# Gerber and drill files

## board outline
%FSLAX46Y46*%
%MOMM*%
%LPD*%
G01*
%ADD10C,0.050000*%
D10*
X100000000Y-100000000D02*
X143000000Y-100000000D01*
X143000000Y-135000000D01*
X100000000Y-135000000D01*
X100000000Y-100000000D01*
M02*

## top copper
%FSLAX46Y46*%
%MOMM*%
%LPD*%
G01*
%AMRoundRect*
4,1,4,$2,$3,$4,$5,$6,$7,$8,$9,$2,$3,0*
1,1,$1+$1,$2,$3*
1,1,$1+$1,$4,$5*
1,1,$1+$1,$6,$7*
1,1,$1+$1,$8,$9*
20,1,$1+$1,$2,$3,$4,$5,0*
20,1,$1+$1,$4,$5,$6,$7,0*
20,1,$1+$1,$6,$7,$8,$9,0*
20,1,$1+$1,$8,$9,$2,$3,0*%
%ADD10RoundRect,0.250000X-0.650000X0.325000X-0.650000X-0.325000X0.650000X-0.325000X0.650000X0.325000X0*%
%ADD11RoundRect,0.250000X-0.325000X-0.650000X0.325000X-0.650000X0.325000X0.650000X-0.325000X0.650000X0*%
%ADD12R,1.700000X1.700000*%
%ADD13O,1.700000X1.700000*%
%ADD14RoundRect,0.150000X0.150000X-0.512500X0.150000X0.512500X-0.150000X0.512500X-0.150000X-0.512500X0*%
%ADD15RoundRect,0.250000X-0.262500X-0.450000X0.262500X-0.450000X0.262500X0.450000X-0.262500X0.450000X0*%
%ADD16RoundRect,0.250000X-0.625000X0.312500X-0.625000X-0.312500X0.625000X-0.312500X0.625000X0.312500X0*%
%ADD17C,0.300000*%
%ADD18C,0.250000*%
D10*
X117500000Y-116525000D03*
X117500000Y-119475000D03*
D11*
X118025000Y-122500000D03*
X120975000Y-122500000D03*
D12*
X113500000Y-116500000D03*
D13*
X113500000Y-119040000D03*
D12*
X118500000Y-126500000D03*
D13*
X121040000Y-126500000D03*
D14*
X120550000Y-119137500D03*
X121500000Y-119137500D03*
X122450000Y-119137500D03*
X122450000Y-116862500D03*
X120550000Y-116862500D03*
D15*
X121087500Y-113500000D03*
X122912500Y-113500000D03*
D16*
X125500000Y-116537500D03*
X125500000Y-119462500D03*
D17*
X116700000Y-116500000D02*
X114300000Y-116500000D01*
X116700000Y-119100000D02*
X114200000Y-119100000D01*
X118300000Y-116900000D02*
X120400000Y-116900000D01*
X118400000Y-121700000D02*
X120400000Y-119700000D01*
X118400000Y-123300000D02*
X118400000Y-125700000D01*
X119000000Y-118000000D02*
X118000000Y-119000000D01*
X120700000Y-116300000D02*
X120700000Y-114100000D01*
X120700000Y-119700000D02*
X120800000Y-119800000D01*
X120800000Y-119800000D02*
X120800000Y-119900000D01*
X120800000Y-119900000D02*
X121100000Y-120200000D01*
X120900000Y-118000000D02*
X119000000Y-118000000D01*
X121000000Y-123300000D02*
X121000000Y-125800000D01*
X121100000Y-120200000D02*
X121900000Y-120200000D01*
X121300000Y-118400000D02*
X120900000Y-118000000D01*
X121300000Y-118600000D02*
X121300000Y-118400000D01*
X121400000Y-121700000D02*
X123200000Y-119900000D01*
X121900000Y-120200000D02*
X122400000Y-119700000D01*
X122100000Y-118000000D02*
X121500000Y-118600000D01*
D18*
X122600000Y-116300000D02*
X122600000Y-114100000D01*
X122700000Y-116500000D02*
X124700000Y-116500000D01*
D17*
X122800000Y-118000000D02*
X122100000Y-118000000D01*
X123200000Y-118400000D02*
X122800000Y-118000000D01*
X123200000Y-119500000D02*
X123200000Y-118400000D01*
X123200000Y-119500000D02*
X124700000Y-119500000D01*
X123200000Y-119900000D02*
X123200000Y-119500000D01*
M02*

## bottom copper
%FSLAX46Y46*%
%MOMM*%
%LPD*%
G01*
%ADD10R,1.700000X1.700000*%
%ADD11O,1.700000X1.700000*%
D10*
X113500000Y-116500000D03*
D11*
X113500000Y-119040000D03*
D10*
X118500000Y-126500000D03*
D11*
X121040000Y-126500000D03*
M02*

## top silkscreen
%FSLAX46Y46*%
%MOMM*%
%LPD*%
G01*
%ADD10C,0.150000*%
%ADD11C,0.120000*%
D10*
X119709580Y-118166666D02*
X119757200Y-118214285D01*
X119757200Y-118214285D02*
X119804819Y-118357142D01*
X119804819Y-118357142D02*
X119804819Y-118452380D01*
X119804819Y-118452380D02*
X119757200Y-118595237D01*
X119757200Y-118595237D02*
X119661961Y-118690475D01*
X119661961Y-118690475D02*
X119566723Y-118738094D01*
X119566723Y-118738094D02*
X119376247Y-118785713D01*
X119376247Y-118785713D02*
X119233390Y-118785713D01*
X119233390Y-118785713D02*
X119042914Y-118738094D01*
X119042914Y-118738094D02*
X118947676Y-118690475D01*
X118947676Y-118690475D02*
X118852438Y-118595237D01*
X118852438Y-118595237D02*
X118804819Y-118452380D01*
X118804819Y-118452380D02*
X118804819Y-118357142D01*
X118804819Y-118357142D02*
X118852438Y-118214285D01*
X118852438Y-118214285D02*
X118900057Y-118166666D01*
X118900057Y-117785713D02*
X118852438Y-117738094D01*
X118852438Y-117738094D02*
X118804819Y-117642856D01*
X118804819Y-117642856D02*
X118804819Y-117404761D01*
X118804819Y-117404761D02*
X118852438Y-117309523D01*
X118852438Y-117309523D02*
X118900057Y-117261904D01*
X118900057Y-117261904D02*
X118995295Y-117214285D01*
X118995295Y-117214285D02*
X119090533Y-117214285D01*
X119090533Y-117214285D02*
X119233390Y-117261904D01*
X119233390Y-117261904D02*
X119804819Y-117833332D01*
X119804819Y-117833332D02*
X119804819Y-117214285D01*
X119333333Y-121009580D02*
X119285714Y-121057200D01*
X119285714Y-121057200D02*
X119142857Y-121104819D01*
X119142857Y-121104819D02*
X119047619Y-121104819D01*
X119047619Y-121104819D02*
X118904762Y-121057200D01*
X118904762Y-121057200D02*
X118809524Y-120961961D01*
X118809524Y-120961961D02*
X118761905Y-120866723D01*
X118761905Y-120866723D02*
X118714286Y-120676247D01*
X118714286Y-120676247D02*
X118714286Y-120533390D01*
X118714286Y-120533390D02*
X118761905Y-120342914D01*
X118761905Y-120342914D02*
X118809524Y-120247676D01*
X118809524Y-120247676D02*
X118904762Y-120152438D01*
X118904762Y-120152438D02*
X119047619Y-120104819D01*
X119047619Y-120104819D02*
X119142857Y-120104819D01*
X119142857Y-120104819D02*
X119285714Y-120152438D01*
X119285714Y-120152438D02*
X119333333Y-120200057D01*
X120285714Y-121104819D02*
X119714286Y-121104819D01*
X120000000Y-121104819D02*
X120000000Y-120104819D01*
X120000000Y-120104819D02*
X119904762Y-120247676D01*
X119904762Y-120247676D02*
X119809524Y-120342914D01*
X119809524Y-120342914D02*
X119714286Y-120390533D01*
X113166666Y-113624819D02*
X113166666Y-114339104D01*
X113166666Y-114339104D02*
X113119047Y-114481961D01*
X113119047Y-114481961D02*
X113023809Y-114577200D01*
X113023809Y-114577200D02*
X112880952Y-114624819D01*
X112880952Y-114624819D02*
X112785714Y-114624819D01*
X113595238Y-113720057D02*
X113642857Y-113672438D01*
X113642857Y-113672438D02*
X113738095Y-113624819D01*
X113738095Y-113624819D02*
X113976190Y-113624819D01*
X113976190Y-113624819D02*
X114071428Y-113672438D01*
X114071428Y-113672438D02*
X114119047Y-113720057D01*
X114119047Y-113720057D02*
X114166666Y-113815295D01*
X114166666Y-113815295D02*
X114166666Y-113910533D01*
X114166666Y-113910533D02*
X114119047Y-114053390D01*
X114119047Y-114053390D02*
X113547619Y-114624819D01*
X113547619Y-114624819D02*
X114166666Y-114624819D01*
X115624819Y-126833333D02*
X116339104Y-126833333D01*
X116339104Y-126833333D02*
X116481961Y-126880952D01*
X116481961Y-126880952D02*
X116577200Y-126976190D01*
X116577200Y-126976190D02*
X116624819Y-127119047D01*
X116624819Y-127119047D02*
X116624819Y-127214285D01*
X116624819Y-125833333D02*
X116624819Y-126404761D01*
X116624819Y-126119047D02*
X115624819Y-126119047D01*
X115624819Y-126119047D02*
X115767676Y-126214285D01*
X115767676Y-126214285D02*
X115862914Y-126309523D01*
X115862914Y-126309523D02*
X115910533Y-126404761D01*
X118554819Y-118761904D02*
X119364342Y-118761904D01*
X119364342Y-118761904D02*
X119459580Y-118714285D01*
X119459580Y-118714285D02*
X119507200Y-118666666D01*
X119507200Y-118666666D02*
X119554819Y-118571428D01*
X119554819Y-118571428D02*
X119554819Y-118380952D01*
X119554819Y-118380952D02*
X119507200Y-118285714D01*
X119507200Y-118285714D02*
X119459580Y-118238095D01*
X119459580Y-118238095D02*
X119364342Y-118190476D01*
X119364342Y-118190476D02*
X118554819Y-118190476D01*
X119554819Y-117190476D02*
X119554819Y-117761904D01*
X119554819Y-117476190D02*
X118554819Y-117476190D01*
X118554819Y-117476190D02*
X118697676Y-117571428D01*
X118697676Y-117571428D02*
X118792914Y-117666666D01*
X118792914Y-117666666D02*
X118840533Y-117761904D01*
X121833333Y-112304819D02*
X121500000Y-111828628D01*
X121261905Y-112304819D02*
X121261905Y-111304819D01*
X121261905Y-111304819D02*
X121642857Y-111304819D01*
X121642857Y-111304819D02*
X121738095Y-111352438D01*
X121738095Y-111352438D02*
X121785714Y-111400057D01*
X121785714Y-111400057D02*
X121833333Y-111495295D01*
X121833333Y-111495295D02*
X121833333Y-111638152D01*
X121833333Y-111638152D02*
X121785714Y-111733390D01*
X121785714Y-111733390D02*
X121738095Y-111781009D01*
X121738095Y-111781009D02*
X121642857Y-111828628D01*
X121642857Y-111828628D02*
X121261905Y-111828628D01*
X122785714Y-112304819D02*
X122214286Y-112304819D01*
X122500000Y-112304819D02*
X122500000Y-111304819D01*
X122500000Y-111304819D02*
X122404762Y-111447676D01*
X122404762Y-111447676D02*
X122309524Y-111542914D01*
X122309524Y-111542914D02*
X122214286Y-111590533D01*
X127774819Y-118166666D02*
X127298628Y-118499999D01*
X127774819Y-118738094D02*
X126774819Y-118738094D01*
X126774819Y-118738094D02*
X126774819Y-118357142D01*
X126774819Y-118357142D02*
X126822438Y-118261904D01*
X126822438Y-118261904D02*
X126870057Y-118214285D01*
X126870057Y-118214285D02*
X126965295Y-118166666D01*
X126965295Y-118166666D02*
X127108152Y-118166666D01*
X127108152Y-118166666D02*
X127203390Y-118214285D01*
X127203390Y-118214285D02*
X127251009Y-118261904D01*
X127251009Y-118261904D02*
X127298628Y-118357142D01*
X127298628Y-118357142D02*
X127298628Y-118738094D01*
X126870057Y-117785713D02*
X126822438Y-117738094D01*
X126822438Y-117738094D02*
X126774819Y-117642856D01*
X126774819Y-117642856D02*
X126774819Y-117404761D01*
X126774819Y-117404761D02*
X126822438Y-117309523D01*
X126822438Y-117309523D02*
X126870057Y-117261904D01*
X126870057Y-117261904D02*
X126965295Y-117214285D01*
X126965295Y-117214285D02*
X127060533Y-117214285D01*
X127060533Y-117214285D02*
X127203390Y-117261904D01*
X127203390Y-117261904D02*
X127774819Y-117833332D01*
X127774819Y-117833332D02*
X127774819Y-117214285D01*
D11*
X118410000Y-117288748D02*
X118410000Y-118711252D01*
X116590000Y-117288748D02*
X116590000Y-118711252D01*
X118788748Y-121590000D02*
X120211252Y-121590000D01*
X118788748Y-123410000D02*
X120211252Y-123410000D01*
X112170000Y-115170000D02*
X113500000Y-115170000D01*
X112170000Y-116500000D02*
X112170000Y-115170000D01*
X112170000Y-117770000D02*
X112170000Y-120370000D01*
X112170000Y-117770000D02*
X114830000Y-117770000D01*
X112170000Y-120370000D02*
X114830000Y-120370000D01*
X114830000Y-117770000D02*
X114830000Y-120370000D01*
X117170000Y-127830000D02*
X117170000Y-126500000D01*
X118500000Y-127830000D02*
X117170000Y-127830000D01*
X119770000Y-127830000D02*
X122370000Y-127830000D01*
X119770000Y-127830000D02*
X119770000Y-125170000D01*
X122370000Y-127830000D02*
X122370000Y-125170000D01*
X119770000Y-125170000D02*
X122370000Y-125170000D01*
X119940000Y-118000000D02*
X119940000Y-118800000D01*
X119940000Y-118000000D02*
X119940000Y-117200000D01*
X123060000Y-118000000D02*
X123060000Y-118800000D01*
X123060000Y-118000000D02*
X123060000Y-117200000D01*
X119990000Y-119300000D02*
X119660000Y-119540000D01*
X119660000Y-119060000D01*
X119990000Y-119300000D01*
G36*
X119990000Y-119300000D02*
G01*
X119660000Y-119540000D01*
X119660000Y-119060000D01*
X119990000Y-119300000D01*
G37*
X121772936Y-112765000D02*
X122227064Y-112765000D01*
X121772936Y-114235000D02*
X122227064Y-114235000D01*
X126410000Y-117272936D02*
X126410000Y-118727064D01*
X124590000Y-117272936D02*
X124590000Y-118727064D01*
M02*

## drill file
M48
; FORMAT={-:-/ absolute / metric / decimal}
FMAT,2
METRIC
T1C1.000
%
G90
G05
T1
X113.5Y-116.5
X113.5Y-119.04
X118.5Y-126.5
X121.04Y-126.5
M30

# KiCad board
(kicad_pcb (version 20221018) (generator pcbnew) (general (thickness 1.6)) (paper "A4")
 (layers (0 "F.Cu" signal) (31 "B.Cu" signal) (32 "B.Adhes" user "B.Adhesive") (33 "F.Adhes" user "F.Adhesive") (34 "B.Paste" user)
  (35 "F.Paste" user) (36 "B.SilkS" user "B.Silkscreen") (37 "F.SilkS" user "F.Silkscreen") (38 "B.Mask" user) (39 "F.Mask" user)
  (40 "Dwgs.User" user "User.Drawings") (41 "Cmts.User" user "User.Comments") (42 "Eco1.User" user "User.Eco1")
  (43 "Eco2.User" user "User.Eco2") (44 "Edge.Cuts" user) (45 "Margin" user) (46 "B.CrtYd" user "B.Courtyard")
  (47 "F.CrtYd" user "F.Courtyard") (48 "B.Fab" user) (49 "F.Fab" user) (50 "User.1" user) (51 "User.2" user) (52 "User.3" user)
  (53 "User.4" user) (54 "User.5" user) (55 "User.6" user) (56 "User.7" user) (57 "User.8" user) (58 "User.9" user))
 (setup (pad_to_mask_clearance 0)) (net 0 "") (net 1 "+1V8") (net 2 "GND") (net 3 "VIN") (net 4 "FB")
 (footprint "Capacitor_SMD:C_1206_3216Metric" (layer "F.Cu") (at 117.5 118 -90)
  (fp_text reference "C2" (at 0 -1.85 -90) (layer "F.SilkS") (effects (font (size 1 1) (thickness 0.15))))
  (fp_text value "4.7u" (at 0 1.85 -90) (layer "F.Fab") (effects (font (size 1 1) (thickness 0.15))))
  (fp_line (start -0.711252 -0.91) (end 0.711252 -0.91) (stroke (width 0.12) (type solid)) (layer "F.SilkS"))
  (fp_line (start -0.711252 0.91) (end 0.711252 0.91) (stroke (width 0.12) (type solid)) (layer "F.SilkS"))
  (pad "1" smd roundrect (at -1.475 0 270) (size 1.15 1.8) (layers "F.Cu" "F.Paste" "F.Mask") (roundrect_rratio 0.217391) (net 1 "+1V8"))
  (pad "2" smd roundrect (at 1.475 0 270) (size 1.15 1.8) (layers "F.Cu" "F.Paste" "F.Mask") (roundrect_rratio 0.217391) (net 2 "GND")))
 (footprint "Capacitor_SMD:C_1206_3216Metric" (layer "F.Cu") (at 119.5 122.5)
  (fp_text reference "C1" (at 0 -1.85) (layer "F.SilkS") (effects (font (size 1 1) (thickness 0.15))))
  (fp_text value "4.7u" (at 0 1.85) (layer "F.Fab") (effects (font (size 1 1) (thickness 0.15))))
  (fp_line (start -0.711252 -0.91) (end 0.711252 -0.91) (stroke (width 0.12) (type solid)) (layer "F.SilkS"))
  (fp_line (start -0.711252 0.91) (end 0.711252 0.91) (stroke (width 0.12) (type solid)) (layer "F.SilkS"))
  (pad "1" smd roundrect (at -1.475 0) (size 1.15 1.8) (layers "F.Cu" "F.Paste" "F.Mask") (roundrect_rratio 0.217391) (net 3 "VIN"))
  (pad "2" smd roundrect (at 1.475 0) (size 1.15 1.8) (layers "F.Cu" "F.Paste" "F.Mask") (roundrect_rratio 0.217391) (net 2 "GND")))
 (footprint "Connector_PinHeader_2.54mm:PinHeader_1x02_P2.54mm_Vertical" (layer "F.Cu") (at 113.5 116.5)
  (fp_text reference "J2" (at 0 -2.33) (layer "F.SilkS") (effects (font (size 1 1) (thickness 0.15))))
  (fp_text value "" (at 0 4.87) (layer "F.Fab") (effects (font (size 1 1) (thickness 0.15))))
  (fp_line (start -1.33 -1.33) (end 0 -1.33) (stroke (width 0.12) (type solid)) (layer "F.SilkS"))
  (fp_line (start -1.33 0) (end -1.33 -1.33) (stroke (width 0.12) (type solid)) (layer "F.SilkS"))
  (fp_line (start -1.33 1.27) (end -1.33 3.87) (stroke (width 0.12) (type solid)) (layer "F.SilkS"))
  (fp_line (start -1.33 1.27) (end 1.33 1.27) (stroke (width 0.12) (type solid)) (layer "F.SilkS"))
  (fp_line (start -1.33 3.87) (end 1.33 3.87) (stroke (width 0.12) (type solid)) (layer "F.SilkS"))
  (fp_line (start 1.33 1.27) (end 1.33 3.87) (stroke (width 0.12) (type solid)) (layer "F.SilkS"))
  (pad "1" thru_hole rect (at 0 0) (size 1.7 1.7) (drill 1) (layers "*.Cu" "*.Mask") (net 1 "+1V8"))
  (pad "2" thru_hole oval (at 0 2.54) (size 1.7 1.7) (drill 1) (layers "*.Cu" "*.Mask") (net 2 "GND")))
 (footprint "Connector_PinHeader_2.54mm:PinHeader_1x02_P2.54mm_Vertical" (layer "F.Cu") (at 118.5 126.5 90)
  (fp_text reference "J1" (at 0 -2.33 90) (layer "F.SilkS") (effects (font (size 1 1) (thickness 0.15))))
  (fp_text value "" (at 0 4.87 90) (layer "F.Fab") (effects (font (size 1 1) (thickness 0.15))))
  (fp_line (start -1.33 -1.33) (end 0 -1.33) (stroke (width 0.12) (type solid)) (layer "F.SilkS"))
  (fp_line (start -1.33 0) (end -1.33 -1.33) (stroke (width 0.12) (type solid)) (layer "F.SilkS"))
  (fp_line (start -1.33 1.27) (end -1.33 3.87) (stroke (width 0.12) (type solid)) (layer "F.SilkS"))
  (fp_line (start -1.33 1.27) (end 1.33 1.27) (stroke (width 0.12) (type solid)) (layer "F.SilkS"))
  (fp_line (start -1.33 3.87) (end 1.33 3.87) (stroke (width 0.12) (type solid)) (layer "F.SilkS"))
  (fp_line (start 1.33 1.27) (end 1.33 3.87) (stroke (width 0.12) (type solid)) (layer "F.SilkS"))
  (pad "1" thru_hole rect (at 0 0 90) (size 1.7 1.7) (drill 1) (layers "*.Cu" "*.Mask") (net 3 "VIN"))
  (pad "2" thru_hole oval (at 0 2.54 90) (size 1.7 1.7) (drill 1) (layers "*.Cu" "*.Mask") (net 2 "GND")))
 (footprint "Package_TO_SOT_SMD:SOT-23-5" (layer "F.Cu") (at 121.5 118 90)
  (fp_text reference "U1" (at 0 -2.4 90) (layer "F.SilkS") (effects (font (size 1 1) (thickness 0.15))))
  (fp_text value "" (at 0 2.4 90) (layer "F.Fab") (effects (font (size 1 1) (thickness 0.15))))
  (fp_line (start 0 -1.56) (end -0.8 -1.56) (stroke (width 0.12) (type solid)) (layer "F.SilkS"))
  (fp_line (start 0 -1.56) (end 0.8 -1.56) (stroke (width 0.12) (type solid)) (layer "F.SilkS"))
  (fp_line (start 0 1.56) (end -0.8 1.56) (stroke (width 0.12) (type solid)) (layer "F.SilkS"))
  (fp_line (start 0 1.56) (end 0.8 1.56) (stroke (width 0.12) (type solid)) (layer "F.SilkS"))
  (fp_poly
   (pts (xy -1.3 -1.51) (xy -1.54 -1.84) (xy -1.06 -1.84) (xy -1.3 -1.51)) (stroke (width 0.12) (type solid)) (fill solid) (layer "F.SilkS"))
  (pad "1" smd roundrect (at -1.1375 -0.95 90) (size 1.325 0.6) (layers "F.Cu" "F.Paste" "F.Mask") (roundrect_rratio 0.25) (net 3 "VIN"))
  (pad "2" smd roundrect (at -1.1375 0 90) (size 1.325 0.6) (layers "F.Cu" "F.Paste" "F.Mask") (roundrect_rratio 0.25) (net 2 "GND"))
  (pad "3" smd roundrect (at -1.1375 0.95 90) (size 1.325 0.6) (layers "F.Cu" "F.Paste" "F.Mask") (roundrect_rratio 0.25) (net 3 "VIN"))
  (pad "4" smd roundrect (at 1.1375 0.95 90) (size 1.325 0.6) (layers "F.Cu" "F.Paste" "F.Mask") (roundrect_rratio 0.25) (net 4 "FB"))
  (pad "5" smd roundrect (at 1.1375 -0.95 90) (size 1.325 0.6) (layers "F.Cu" "F.Paste" "F.Mask") (roundrect_rratio 0.25) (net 1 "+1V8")))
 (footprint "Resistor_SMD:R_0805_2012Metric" (layer "F.Cu") (at 122 113.5)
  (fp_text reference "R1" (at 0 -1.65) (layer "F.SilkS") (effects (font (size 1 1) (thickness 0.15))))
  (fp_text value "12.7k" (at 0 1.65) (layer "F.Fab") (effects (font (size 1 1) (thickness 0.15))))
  (fp_line (start -0.227064 -0.735) (end 0.227064 -0.735) (stroke (width 0.12) (type solid)) (layer "F.SilkS"))
  (fp_line (start -0.227064 0.735) (end 0.227064 0.735) (stroke (width 0.12) (type solid)) (layer "F.SilkS"))
  (pad "1" smd roundrect (at -0.9125 0) (size 1.025 1.4) (layers "F.Cu" "F.Paste" "F.Mask") (roundrect_rratio 0.243902) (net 1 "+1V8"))
  (pad "2" smd roundrect (at 0.9125 0) (size 1.025 1.4) (layers "F.Cu" "F.Paste" "F.Mask") (roundrect_rratio 0.243902) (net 4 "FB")))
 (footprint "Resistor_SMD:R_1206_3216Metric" (layer "F.Cu") (at 125.5 118 -90)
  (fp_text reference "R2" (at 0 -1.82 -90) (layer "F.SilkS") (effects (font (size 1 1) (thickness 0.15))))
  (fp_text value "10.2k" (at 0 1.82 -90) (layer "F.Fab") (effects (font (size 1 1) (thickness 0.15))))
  (fp_line (start -0.727064 -0.91) (end 0.727064 -0.91) (stroke (width 0.12) (type solid)) (layer "F.SilkS"))
  (fp_line (start -0.727064 0.91) (end 0.727064 0.91) (stroke (width 0.12) (type solid)) (layer "F.SilkS"))
  (pad "1" smd roundrect (at -1.4625 0 270) (size 1.125 1.75) (layers "F.Cu" "F.Paste" "F.Mask") (roundrect_rratio 0.222222) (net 4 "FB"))
  (pad "2" smd roundrect (at 1.4625 0 270) (size 1.125 1.75) (layers "F.Cu" "F.Paste" "F.Mask") (roundrect_rratio 0.222222) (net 2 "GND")))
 (gr_rect (start 100 100) (end 143 135) (stroke (width 0.05) (type default)) (fill none) (layer "Edge.Cuts"))
 (segment (start 116.7 116.5) (end 114.3 116.5) (width 0.3) (layer "F.Cu") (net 1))
 (segment (start 116.7 119.1) (end 114.2 119.1) (width 0.3) (layer "F.Cu") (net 2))
 (segment (start 118.3 116.9) (end 120.4 116.9) (width 0.3) (layer "F.Cu") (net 1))
 (segment (start 118.4 121.7) (end 120.4 119.7) (width 0.3) (layer "F.Cu") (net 3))
 (segment (start 118.4 123.3) (end 118.4 125.7) (width 0.3) (layer "F.Cu") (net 3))
 (segment (start 119 118) (end 118 119) (width 0.3) (layer "F.Cu") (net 2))
 (segment (start 120.7 116.3) (end 120.7 114.1) (width 0.3) (layer "F.Cu") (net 1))
 (segment (start 120.7 119.7) (end 120.8 119.8) (width 0.3) (layer "F.Cu") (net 3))
 (segment (start 120.8 119.8) (end 120.8 119.9) (width 0.3) (layer "F.Cu") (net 3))
 (segment (start 120.8 119.9) (end 121.1 120.2) (width 0.3) (layer "F.Cu") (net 3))
 (segment (start 120.9 118) (end 119 118) (width 0.3) (layer "F.Cu") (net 2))
 (segment (start 121 123.3) (end 121 125.8) (width 0.3) (layer "F.Cu") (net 2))
 (segment (start 121.1 120.2) (end 121.9 120.2) (width 0.3) (layer "F.Cu") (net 3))
 (segment (start 121.3 118.4) (end 120.9 118) (width 0.3) (layer "F.Cu") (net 2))
 (segment (start 121.3 118.6) (end 121.3 118.4) (width 0.3) (layer "F.Cu") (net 2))
 (segment (start 121.4 121.7) (end 123.2 119.9) (width 0.3) (layer "F.Cu") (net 2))
 (segment (start 121.9 120.2) (end 122.4 119.7) (width 0.3) (layer "F.Cu") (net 3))
 (segment (start 122.1 118) (end 121.5 118.6) (width 0.3) (layer "F.Cu") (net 2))
 (segment (start 122.6 116.3) (end 122.6 114.1) (width 0.25) (layer "F.Cu") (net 4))
 (segment (start 122.7 116.5) (end 124.7 116.5) (width 0.25) (layer "F.Cu") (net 4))
 (segment (start 122.8 118) (end 122.1 118) (width 0.3) (layer "F.Cu") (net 2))
 (segment (start 123.2 118.4) (end 122.8 118) (width 0.3) (layer "F.Cu") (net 2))
 (segment (start 123.2 119.5) (end 123.2 118.4) (width 0.3) (layer "F.Cu") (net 2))
 (segment (start 123.2 119.5) (end 124.7 119.5) (width 0.3) (layer "F.Cu") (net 2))
 (segment (start 123.2 119.9) (end 123.2 119.5) (width 0.3) (layer "F.Cu") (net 2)))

